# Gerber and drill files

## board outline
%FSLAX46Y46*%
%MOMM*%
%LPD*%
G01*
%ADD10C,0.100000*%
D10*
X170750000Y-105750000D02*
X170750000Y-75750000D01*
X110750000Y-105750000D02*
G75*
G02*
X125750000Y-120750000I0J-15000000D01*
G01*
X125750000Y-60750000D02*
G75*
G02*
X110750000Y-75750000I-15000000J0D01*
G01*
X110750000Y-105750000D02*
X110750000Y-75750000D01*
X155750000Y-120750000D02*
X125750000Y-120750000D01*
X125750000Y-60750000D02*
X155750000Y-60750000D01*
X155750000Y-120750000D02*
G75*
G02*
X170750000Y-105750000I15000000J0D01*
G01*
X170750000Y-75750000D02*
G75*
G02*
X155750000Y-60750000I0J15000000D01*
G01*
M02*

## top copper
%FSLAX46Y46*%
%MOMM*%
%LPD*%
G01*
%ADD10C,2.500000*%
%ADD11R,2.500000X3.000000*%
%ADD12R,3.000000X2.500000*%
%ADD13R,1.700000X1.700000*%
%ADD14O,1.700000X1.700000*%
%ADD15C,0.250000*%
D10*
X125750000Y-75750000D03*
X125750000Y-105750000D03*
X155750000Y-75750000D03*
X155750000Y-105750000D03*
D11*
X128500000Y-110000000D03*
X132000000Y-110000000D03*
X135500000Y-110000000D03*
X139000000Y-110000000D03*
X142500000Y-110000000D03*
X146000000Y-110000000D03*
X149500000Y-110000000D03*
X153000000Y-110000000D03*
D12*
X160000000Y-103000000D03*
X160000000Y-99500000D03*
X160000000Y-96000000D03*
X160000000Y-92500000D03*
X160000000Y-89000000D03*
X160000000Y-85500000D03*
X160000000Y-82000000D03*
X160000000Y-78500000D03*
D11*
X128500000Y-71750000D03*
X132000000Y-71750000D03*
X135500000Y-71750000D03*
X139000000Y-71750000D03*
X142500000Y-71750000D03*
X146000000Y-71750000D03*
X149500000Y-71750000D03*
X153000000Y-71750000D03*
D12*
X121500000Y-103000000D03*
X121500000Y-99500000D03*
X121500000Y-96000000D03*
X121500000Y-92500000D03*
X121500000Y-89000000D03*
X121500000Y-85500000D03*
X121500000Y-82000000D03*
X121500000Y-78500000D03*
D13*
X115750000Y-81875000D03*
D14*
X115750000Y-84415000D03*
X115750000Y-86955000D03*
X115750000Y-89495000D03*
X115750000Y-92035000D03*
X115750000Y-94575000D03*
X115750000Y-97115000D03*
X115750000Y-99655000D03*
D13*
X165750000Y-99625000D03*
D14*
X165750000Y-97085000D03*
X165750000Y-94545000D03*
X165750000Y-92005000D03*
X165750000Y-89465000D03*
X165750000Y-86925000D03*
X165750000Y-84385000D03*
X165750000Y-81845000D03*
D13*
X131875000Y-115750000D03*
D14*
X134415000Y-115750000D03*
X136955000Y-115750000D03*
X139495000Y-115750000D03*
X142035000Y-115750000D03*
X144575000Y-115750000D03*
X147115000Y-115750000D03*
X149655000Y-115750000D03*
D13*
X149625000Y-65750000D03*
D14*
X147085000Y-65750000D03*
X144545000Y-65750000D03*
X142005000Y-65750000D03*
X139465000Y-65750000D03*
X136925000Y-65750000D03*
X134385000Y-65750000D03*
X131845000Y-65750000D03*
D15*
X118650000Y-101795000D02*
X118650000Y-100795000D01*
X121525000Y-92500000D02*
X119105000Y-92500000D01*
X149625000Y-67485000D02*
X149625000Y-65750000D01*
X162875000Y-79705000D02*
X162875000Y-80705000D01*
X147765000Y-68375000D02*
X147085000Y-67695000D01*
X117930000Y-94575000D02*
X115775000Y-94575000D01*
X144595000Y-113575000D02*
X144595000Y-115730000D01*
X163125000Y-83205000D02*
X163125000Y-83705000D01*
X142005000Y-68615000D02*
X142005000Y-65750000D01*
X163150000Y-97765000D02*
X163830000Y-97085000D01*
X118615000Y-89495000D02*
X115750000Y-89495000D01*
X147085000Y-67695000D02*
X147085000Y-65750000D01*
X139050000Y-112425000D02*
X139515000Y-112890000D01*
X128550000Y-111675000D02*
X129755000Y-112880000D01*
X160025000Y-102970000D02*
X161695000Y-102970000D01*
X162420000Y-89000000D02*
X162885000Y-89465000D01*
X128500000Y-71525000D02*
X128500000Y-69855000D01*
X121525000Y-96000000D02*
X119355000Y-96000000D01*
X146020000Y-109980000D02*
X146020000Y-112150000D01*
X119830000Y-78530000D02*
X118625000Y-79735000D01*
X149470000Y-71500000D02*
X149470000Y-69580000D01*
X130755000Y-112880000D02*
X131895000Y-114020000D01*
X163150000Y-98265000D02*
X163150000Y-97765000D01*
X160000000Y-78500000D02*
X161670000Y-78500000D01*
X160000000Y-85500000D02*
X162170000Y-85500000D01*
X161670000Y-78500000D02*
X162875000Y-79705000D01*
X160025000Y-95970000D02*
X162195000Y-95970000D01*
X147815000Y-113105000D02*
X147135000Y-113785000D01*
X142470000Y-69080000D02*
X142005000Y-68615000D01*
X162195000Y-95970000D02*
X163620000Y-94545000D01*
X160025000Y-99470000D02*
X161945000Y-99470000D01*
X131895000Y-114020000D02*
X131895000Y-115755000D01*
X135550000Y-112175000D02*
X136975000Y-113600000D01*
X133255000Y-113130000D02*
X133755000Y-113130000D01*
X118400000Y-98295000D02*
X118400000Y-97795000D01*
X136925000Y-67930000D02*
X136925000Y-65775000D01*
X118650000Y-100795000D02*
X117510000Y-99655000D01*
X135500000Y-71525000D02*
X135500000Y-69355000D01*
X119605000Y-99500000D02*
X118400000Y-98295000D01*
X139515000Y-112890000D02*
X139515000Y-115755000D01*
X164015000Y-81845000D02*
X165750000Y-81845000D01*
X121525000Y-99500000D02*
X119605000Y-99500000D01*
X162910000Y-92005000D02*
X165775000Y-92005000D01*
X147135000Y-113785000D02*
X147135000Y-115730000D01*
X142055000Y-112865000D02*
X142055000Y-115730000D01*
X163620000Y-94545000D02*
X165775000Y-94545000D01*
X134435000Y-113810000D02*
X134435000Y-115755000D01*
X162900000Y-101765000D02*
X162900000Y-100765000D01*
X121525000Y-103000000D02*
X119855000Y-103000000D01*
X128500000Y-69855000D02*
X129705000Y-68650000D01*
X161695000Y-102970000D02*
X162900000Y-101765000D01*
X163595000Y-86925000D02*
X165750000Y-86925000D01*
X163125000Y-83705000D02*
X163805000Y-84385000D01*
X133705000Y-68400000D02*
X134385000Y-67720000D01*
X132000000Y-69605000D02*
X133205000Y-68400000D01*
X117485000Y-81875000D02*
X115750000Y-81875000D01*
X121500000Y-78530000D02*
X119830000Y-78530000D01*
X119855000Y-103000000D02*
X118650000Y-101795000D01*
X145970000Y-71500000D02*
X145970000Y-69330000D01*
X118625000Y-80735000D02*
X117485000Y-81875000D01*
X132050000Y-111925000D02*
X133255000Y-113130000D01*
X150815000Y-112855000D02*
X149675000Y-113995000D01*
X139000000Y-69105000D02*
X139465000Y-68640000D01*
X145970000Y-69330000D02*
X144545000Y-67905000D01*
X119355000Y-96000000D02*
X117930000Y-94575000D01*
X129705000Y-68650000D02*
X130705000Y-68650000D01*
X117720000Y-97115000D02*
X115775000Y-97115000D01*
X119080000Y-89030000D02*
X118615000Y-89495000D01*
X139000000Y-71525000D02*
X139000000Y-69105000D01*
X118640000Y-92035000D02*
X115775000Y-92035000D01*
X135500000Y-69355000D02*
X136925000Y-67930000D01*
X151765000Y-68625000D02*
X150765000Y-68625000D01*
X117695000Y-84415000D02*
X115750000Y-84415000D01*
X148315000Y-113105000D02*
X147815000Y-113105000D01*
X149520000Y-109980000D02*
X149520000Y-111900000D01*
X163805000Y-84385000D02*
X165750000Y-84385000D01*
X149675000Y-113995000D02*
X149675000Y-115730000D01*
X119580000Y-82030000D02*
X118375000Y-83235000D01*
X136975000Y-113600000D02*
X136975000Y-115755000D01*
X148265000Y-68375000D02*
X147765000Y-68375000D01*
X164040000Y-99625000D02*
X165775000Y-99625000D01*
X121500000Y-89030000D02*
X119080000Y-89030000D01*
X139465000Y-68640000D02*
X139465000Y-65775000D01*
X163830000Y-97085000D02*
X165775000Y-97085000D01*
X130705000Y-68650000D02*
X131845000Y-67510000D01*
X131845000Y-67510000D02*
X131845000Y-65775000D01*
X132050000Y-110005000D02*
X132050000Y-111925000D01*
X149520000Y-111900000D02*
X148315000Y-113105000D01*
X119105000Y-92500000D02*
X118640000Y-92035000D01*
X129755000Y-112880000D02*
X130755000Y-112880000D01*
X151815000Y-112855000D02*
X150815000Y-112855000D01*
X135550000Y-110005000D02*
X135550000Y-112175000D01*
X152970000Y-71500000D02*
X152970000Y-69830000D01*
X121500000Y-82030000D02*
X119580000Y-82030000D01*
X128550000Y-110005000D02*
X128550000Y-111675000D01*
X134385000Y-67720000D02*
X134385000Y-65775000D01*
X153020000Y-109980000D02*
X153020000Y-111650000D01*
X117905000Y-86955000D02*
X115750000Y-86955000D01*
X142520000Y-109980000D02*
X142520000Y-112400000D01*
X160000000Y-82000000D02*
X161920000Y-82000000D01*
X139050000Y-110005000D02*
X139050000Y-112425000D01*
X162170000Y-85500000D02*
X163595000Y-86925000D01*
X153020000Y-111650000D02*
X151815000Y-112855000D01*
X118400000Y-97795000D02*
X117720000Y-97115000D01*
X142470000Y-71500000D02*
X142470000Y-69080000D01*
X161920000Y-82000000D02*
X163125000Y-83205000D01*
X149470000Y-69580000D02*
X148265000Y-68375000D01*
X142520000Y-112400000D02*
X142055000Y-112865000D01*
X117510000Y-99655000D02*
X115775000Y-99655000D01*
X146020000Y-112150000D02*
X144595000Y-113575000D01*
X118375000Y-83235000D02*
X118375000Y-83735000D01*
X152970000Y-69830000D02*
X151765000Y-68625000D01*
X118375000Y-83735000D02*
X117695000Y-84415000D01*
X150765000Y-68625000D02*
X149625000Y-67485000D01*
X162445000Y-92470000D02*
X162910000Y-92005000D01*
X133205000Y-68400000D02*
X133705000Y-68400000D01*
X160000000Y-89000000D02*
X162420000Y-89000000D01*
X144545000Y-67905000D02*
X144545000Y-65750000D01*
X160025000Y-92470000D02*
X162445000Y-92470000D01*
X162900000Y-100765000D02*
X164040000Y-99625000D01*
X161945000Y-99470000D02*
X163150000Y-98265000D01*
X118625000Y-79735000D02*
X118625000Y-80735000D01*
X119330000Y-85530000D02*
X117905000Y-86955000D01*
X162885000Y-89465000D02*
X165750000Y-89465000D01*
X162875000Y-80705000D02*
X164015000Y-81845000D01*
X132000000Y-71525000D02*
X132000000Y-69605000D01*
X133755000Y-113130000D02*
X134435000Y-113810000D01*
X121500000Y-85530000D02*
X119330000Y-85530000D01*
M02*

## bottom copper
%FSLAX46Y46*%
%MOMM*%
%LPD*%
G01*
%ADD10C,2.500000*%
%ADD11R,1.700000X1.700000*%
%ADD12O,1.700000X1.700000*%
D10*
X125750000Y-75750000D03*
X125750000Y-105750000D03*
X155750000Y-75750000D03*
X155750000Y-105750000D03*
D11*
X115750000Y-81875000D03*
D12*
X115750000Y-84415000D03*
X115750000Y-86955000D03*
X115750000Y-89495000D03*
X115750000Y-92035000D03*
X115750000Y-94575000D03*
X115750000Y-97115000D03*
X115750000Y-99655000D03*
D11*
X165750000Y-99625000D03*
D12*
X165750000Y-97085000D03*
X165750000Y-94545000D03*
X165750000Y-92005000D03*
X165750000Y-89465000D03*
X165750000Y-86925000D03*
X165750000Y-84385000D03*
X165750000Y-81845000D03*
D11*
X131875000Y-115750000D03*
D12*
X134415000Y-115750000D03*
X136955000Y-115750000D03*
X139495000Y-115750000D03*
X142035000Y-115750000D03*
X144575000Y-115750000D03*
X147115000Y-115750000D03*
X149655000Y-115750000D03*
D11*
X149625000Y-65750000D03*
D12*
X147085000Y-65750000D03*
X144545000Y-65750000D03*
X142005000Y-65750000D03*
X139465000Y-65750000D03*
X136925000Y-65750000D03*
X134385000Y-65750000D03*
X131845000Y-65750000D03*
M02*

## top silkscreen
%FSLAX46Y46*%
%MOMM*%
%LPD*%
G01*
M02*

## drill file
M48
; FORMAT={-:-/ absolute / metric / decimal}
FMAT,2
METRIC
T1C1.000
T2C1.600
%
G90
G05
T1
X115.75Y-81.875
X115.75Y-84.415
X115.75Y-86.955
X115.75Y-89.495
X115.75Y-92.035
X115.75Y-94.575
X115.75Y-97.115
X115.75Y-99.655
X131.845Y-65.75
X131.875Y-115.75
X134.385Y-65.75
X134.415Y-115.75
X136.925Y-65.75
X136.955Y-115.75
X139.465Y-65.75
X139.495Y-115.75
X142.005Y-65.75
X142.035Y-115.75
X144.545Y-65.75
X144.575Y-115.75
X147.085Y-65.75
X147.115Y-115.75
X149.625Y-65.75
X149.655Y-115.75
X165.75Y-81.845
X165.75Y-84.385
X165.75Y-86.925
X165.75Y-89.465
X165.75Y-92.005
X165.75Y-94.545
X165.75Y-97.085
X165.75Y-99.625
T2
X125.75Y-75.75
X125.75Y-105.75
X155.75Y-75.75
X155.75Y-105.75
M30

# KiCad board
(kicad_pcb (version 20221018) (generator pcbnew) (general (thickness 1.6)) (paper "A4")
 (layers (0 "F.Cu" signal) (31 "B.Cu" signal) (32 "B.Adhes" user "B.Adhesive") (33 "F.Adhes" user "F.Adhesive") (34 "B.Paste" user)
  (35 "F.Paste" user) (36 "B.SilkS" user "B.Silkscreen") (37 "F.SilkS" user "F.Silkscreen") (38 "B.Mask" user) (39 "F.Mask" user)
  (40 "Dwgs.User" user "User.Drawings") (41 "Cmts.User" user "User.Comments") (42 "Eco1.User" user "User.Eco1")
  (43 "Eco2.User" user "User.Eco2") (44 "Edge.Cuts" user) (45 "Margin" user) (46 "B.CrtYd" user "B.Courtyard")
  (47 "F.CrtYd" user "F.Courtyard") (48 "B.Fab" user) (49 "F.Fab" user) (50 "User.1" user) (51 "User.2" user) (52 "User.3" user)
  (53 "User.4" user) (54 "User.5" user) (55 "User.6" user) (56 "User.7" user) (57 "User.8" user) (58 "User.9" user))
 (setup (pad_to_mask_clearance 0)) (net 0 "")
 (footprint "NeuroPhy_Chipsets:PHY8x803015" (layer "F.Cu") (at 140.75 90.75)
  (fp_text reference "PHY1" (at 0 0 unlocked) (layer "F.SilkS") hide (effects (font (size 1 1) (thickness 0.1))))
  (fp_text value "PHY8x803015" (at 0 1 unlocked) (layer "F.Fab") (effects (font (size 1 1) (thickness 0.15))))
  (pad "" thru_hole circle (at -15 -15 90) (size 2.5 2.5) (drill 1.6) (layers "*.Cu" "*.Mask"))
  (pad "" thru_hole circle (at -15 15 90) (size 2.5 2.5) (drill 1.6) (layers "*.Cu" "*.Mask"))
  (pad "" thru_hole circle (at 15 -15 90) (size 2.5 2.5) (drill 1.6) (layers "*.Cu" "*.Mask"))
  (pad "" thru_hole circle (at 15 15 90) (size 2.5 2.5) (drill 1.6) (layers "*.Cu" "*.Mask"))
  (pad "1" smd rect (at -12.25 19.25 90) (size 3 2.5) (layers "F.Cu" "F.Paste" "F.Mask"))
  (pad "2" smd rect (at -8.75 19.25 90) (size 3 2.5) (layers "F.Cu" "F.Paste" "F.Mask"))
  (pad "3" smd rect (at -5.25 19.25 90) (size 3 2.5) (layers "F.Cu" "F.Paste" "F.Mask"))
  (pad "4" smd rect (at -1.75 19.25 90) (size 3 2.5) (layers "F.Cu" "F.Paste" "F.Mask"))
  (pad "5" smd rect (at 1.75 19.25 90) (size 3 2.5) (layers "F.Cu" "F.Paste" "F.Mask"))
  (pad "6" smd rect (at 5.25 19.25 90) (size 3 2.5) (layers "F.Cu" "F.Paste" "F.Mask"))
  (pad "7" smd rect (at 8.75 19.25 90) (size 3 2.5) (layers "F.Cu" "F.Paste" "F.Mask"))
  (pad "8" smd rect (at 12.25 19.25 90) (size 3 2.5) (layers "F.Cu" "F.Paste" "F.Mask"))
  (pad "9" smd rect (at 19.25 12.25 180) (size 3 2.5) (layers "F.Cu" "F.Paste" "F.Mask"))
  (pad "10" smd rect (at 19.25 8.75 180) (size 3 2.5) (layers "F.Cu" "F.Paste" "F.Mask"))
  (pad "11" smd rect (at 19.25 5.25 180) (size 3 2.5) (layers "F.Cu" "F.Paste" "F.Mask"))
  (pad "12" smd rect (at 19.25 1.75 180) (size 3 2.5) (layers "F.Cu" "F.Paste" "F.Mask"))
  (pad "13" smd rect (at 19.25 -1.75 180) (size 3 2.5) (layers "F.Cu" "F.Paste" "F.Mask"))
  (pad "14" smd rect (at 19.25 -5.25 180) (size 3 2.5) (layers "F.Cu" "F.Paste" "F.Mask"))
  (pad "15" smd rect (at 19.25 -8.75 180) (size 3 2.5) (layers "F.Cu" "F.Paste" "F.Mask"))
  (pad "16" smd rect (at 19.25 -12.25 180) (size 3 2.5) (layers "F.Cu" "F.Paste" "F.Mask"))
  (pad "17" smd rect (at -12.25 -19 90) (size 3 2.5) (layers "F.Cu" "F.Paste" "F.Mask"))
  (pad "18" smd rect (at -8.75 -19 90) (size 3 2.5) (layers "F.Cu" "F.Paste" "F.Mask"))
  (pad "19" smd rect (at -5.25 -19 90) (size 3 2.5) (layers "F.Cu" "F.Paste" "F.Mask"))
  (pad "20" smd rect (at -1.75 -19 90) (size 3 2.5) (layers "F.Cu" "F.Paste" "F.Mask"))
  (pad "21" smd rect (at 1.75 -19 90) (size 3 2.5) (layers "F.Cu" "F.Paste" "F.Mask"))
  (pad "22" smd rect (at 5.25 -19 90) (size 3 2.5) (layers "F.Cu" "F.Paste" "F.Mask"))
  (pad "23" smd rect (at 8.75 -19 90) (size 3 2.5) (layers "F.Cu" "F.Paste" "F.Mask"))
  (pad "24" smd rect (at 12.25 -19 90) (size 3 2.5) (layers "F.Cu" "F.Paste" "F.Mask"))
  (pad "25" smd rect (at -19.25 12.25 180) (size 3 2.5) (layers "F.Cu" "F.Paste" "F.Mask"))
  (pad "26" smd rect (at -19.25 8.75 180) (size 3 2.5) (layers "F.Cu" "F.Paste" "F.Mask"))
  (pad "27" smd rect (at -19.25 5.25 180) (size 3 2.5) (layers "F.Cu" "F.Paste" "F.Mask"))
  (pad "28" smd rect (at -19.25 1.75 180) (size 3 2.5) (layers "F.Cu" "F.Paste" "F.Mask"))
  (pad "29" smd rect (at -19.25 -1.75 180) (size 3 2.5) (layers "F.Cu" "F.Paste" "F.Mask"))
  (pad "30" smd rect (at -19.25 -5.25 180) (size 3 2.5) (layers "F.Cu" "F.Paste" "F.Mask"))
  (pad "31" smd rect (at -19.25 -8.75 180) (size 3 2.5) (layers "F.Cu" "F.Paste" "F.Mask"))
  (pad "32" smd rect (at -19.25 -12.25 180) (size 3 2.5) (layers "F.Cu" "F.Paste" "F.Mask")))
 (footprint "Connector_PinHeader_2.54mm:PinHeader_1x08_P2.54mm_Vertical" (layer "B.Cu") (at 115.75 81.875 180)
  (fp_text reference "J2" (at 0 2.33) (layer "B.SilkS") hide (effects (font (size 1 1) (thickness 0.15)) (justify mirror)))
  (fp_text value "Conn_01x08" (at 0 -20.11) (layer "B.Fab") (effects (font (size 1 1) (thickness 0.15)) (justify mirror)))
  (pad "1" thru_hole rect (at 0 0 180) (size 1.7 1.7) (drill 1) (layers "*.Cu" "*.Mask"))
  (pad "2" thru_hole oval (at 0 -2.54 180) (size 1.7 1.7) (drill 1) (layers "*.Cu" "*.Mask"))
  (pad "3" thru_hole oval (at 0 -5.08 180) (size 1.7 1.7) (drill 1) (layers "*.Cu" "*.Mask"))
  (pad "4" thru_hole oval (at 0 -7.62 180) (size 1.7 1.7) (drill 1) (layers "*.Cu" "*.Mask"))
  (pad "5" thru_hole oval (at 0 -10.16 180) (size 1.7 1.7) (drill 1) (layers "*.Cu" "*.Mask"))
  (pad "6" thru_hole oval (at 0 -12.7 180) (size 1.7 1.7) (drill 1) (layers "*.Cu" "*.Mask"))
  (pad "7" thru_hole oval (at 0 -15.24 180) (size 1.7 1.7) (drill 1) (layers "*.Cu" "*.Mask"))
  (pad "8" thru_hole oval (at 0 -17.78 180) (size 1.7 1.7) (drill 1) (layers "*.Cu" "*.Mask")))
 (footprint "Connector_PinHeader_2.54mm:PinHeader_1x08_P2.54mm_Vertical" (layer "B.Cu") (at 165.75 99.625)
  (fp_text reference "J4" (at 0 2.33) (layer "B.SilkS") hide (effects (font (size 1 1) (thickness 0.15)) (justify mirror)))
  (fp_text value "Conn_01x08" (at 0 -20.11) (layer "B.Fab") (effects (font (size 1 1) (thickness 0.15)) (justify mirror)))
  (pad "1" thru_hole rect (at 0 0) (size 1.7 1.7) (drill 1) (layers "*.Cu" "*.Mask"))
  (pad "2" thru_hole oval (at 0 -2.54) (size 1.7 1.7) (drill 1) (layers "*.Cu" "*.Mask"))
  (pad "3" thru_hole oval (at 0 -5.08) (size 1.7 1.7) (drill 1) (layers "*.Cu" "*.Mask"))
  (pad "4" thru_hole oval (at 0 -7.62) (size 1.7 1.7) (drill 1) (layers "*.Cu" "*.Mask"))
  (pad "5" thru_hole oval (at 0 -10.16) (size 1.7 1.7) (drill 1) (layers "*.Cu" "*.Mask"))
  (pad "6" thru_hole oval (at 0 -12.7) (size 1.7 1.7) (drill 1) (layers "*.Cu" "*.Mask"))
  (pad "7" thru_hole oval (at 0 -15.24) (size 1.7 1.7) (drill 1) (layers "*.Cu" "*.Mask"))
  (pad "8" thru_hole oval (at 0 -17.78) (size 1.7 1.7) (drill 1) (layers "*.Cu" "*.Mask")))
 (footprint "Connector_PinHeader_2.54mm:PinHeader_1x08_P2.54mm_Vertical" (layer "B.Cu") (at 131.875 115.75 -90)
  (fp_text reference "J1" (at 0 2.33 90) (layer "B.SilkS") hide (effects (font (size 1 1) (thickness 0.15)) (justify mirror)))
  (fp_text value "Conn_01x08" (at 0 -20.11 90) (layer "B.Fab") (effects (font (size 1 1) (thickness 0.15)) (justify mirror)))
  (pad "1" thru_hole rect (at 0 0 270) (size 1.7 1.7) (drill 1) (layers "*.Cu" "*.Mask"))
  (pad "2" thru_hole oval (at 0 -2.54 270) (size 1.7 1.7) (drill 1) (layers "*.Cu" "*.Mask"))
  (pad "3" thru_hole oval (at 0 -5.08 270) (size 1.7 1.7) (drill 1) (layers "*.Cu" "*.Mask"))
  (pad "4" thru_hole oval (at 0 -7.62 270) (size 1.7 1.7) (drill 1) (layers "*.Cu" "*.Mask"))
  (pad "5" thru_hole oval (at 0 -10.16 270) (size 1.7 1.7) (drill 1) (layers "*.Cu" "*.Mask"))
  (pad "6" thru_hole oval (at 0 -12.7 270) (size 1.7 1.7) (drill 1) (layers "*.Cu" "*.Mask"))
  (pad "7" thru_hole oval (at 0 -15.24 270) (size 1.7 1.7) (drill 1) (layers "*.Cu" "*.Mask"))
  (pad "8" thru_hole oval (at 0 -17.78 270) (size 1.7 1.7) (drill 1) (layers "*.Cu" "*.Mask")))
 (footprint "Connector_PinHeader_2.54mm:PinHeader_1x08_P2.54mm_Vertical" (layer "B.Cu") (at 149.625 65.75 90)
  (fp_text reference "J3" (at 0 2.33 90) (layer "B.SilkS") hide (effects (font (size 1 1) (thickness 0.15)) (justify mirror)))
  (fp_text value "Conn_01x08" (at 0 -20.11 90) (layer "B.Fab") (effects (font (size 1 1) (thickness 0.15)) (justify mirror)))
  (pad "1" thru_hole rect (at 0 0 90) (size 1.7 1.7) (drill 1) (layers "*.Cu" "*.Mask"))
  (pad "2" thru_hole oval (at 0 -2.54 90) (size 1.7 1.7) (drill 1) (layers "*.Cu" "*.Mask"))
  (pad "3" thru_hole oval (at 0 -5.08 90) (size 1.7 1.7) (drill 1) (layers "*.Cu" "*.Mask"))
  (pad "4" thru_hole oval (at 0 -7.62 90) (size 1.7 1.7) (drill 1) (layers "*.Cu" "*.Mask"))
  (pad "5" thru_hole oval (at 0 -10.16 90) (size 1.7 1.7) (drill 1) (layers "*.Cu" "*.Mask"))
  (pad "6" thru_hole oval (at 0 -12.7 90) (size 1.7 1.7) (drill 1) (layers "*.Cu" "*.Mask"))
  (pad "7" thru_hole oval (at 0 -15.24 90) (size 1.7 1.7) (drill 1) (layers "*.Cu" "*.Mask"))
  (pad "8" thru_hole oval (at 0 -17.78 90) (size 1.7 1.7) (drill 1) (layers "*.Cu" "*.Mask")))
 (gr_line (start 170.75 105.75) (end 170.75 75.75) (stroke (width 0.1) (type default)) (layer "Edge.Cuts"))
 (gr_arc (start 110.75 105.75) (mid 121.356602 110.143398) (end 125.75 120.75) (stroke (width 0.1) (type default)) (layer "Edge.Cuts"))
 (gr_arc (start 125.75 60.75) (mid 121.356602 71.356602) (end 110.75 75.75) (stroke (width 0.1) (type default)) (layer "Edge.Cuts"))
 (gr_line (start 110.75 105.75) (end 110.75 75.75) (stroke (width 0.1) (type default)) (layer "Edge.Cuts"))
 (gr_line (start 155.75 120.75) (end 125.75 120.75) (stroke (width 0.1) (type default)) (layer "Edge.Cuts"))
 (gr_line (start 125.75 60.75) (end 155.75 60.75) (stroke (width 0.1) (type default)) (layer "Edge.Cuts"))
 (gr_arc (start 155.75 120.75) (mid 160.143398 110.143398) (end 170.75 105.75) (stroke (width 0.1) (type default)) (layer "Edge.Cuts"))
 (gr_arc (start 170.75 75.75) (mid 160.143398 71.356602) (end 155.75 60.75) (stroke (width 0.1) (type default)) (layer "Edge.Cuts"))
 (segment (start 118.65 101.795) (end 118.65 100.795) (width 0.25) (layer "F.Cu") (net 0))
 (segment (start 121.525 92.5) (end 119.105 92.5) (width 0.25) (layer "F.Cu") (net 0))
 (segment (start 149.625 67.485) (end 149.625 65.75) (width 0.25) (layer "F.Cu") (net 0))
 (segment (start 162.875 79.705) (end 162.875 80.705) (width 0.25) (layer "F.Cu") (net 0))
 (segment (start 147.765 68.375) (end 147.085 67.695) (width 0.25) (layer "F.Cu") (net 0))
 (segment (start 117.93 94.575) (end 115.775 94.575) (width 0.25) (layer "F.Cu") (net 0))
 (segment (start 144.595 113.575) (end 144.595 115.73) (width 0.25) (layer "F.Cu") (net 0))
 (segment (start 163.125 83.205) (end 163.125 83.705) (width 0.25) (layer "F.Cu") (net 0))
 (segment (start 142.005 68.615) (end 142.005 65.75) (width 0.25) (layer "F.Cu") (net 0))
 (segment (start 163.15 97.765) (end 163.83 97.085) (width 0.25) (layer "F.Cu") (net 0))
 (segment (start 118.615 89.495) (end 115.75 89.495) (width 0.25) (layer "F.Cu") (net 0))
 (segment (start 147.085 67.695) (end 147.085 65.75) (width 0.25) (layer "F.Cu") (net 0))
 (segment (start 139.05 112.425) (end 139.515 112.89) (width 0.25) (layer "F.Cu") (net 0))
 (segment (start 128.55 111.675) (end 129.755 112.88) (width 0.25) (layer "F.Cu") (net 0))
 (segment (start 160.025 102.97) (end 161.695 102.97) (width 0.25) (layer "F.Cu") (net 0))
 (segment (start 162.42 89) (end 162.885 89.465) (width 0.25) (layer "F.Cu") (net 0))
 (segment (start 128.5 71.525) (end 128.5 69.855) (width 0.25) (layer "F.Cu") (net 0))
 (segment (start 121.525 96) (end 119.355 96) (width 0.25) (layer "F.Cu") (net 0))
 (segment (start 146.02 109.98) (end 146.02 112.15) (width 0.25) (layer "F.Cu") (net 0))
 (segment (start 119.83 78.53) (end 118.625 79.735) (width 0.25) (layer "F.Cu") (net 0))
 (segment (start 149.47 71.5) (end 149.47 69.58) (width 0.25) (layer "F.Cu") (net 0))
 (segment (start 130.755 112.88) (end 131.895 114.02) (width 0.25) (layer "F.Cu") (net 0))
 (segment (start 163.15 98.265) (end 163.15 97.765) (width 0.25) (layer "F.Cu") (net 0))
 (segment (start 160 78.5) (end 161.67 78.5) (width 0.25) (layer "F.Cu") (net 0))
 (segment (start 160 85.5) (end 162.17 85.5) (width 0.25) (layer "F.Cu") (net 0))
 (segment (start 161.67 78.5) (end 162.875 79.705) (width 0.25) (layer "F.Cu") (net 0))
 (segment (start 160.025 95.97) (end 162.195 95.97) (width 0.25) (layer "F.Cu") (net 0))
 (segment (start 147.815 113.105) (end 147.135 113.785) (width 0.25) (layer "F.Cu") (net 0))
 (segment (start 142.47 69.08) (end 142.005 68.615) (width 0.25) (layer "F.Cu") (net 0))
 (segment (start 162.195 95.97) (end 163.62 94.545) (width 0.25) (layer "F.Cu") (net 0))
 (segment (start 160.025 99.47) (end 161.945 99.47) (width 0.25) (layer "F.Cu") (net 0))
 (segment (start 131.895 114.02) (end 131.895 115.755) (width 0.25) (layer "F.Cu") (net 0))
 (segment (start 135.55 112.175) (end 136.975 113.6) (width 0.25) (layer "F.Cu") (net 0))
 (segment (start 133.255 113.13) (end 133.755 113.13) (width 0.25) (layer "F.Cu") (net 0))
 (segment (start 118.4 98.295) (end 118.4 97.795) (width 0.25) (layer "F.Cu") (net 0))
 (segment (start 136.925 67.93) (end 136.925 65.775) (width 0.25) (layer "F.Cu") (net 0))
 (segment (start 118.65 100.795) (end 117.51 99.655) (width 0.25) (layer "F.Cu") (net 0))
 (segment (start 135.5 71.525) (end 135.5 69.355) (width 0.25) (layer "F.Cu") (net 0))
 (segment (start 119.605 99.5) (end 118.4 98.295) (width 0.25) (layer "F.Cu") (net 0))
 (segment (start 139.515 112.89) (end 139.515 115.755) (width 0.25) (layer "F.Cu") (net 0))
 (segment (start 164.015 81.845) (end 165.75 81.845) (width 0.25) (layer "F.Cu") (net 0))
 (segment (start 121.525 99.5) (end 119.605 99.5) (width 0.25) (layer "F.Cu") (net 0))
 (segment (start 162.91 92.005) (end 165.775 92.005) (width 0.25) (layer "F.Cu") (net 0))
 (segment (start 147.135 113.785) (end 147.135 115.73) (width 0.25) (layer "F.Cu") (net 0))
 (segment (start 142.055 112.865) (end 142.055 115.73) (width 0.25) (layer "F.Cu") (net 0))
 (segment (start 163.62 94.545) (end 165.775 94.545) (width 0.25) (layer "F.Cu") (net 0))
 (segment (start 134.435 113.81) (end 134.435 115.755) (width 0.25) (layer "F.Cu") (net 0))
 (segment (start 162.9 101.765) (end 162.9 100.765) (width 0.25) (layer "F.Cu") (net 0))
 (segment (start 121.525 103) (end 119.855 103) (width 0.25) (layer "F.Cu") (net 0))
 (segment (start 128.5 69.855) (end 129.705 68.65) (width 0.25) (layer "F.Cu") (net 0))
 (segment (start 161.695 102.97) (end 162.9 101.765) (width 0.25) (layer "F.Cu") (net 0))
 (segment (start 163.595 86.925) (end 165.75 86.925) (width 0.25) (layer "F.Cu") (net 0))
 (segment (start 163.125 83.705) (end 163.805 84.385) (width 0.25) (layer "F.Cu") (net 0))
 (segment (start 133.705 68.4) (end 134.385 67.72) (width 0.25) (layer "F.Cu") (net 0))
 (segment (start 132 69.605) (end 133.205 68.4) (width 0.25) (layer "F.Cu") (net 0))
 (segment (start 117.485 81.875) (end 115.75 81.875) (width 0.25) (layer "F.Cu") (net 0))
 (segment (start 121.5 78.53) (end 119.83 78.53) (width 0.25) (layer "F.Cu") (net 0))
 (segment (start 119.855 103) (end 118.65 101.795) (width 0.25) (layer "F.Cu") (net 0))
 (segment (start 145.97 71.5) (end 145.97 69.33) (width 0.25) (layer "F.Cu") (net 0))
 (segment (start 118.625 80.735) (end 117.485 81.875) (width 0.25) (layer "F.Cu") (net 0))
 (segment (start 132.05 111.925) (end 133.255 113.13) (width 0.25) (layer "F.Cu") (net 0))
 (segment (start 150.815 112.855) (end 149.675 113.995) (width 0.25) (layer "F.Cu") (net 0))
 (segment (start 139 69.105) (end 139.465 68.64) (width 0.25) (layer "F.Cu") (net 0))
 (segment (start 145.97 69.33) (end 144.545 67.905) (width 0.25) (layer "F.Cu") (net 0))
 (segment (start 119.355 96) (end 117.93 94.575) (width 0.25) (layer "F.Cu") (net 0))
 (segment (start 129.705 68.65) (end 130.705 68.65) (width 0.25) (layer "F.Cu") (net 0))
 (segment (start 117.72 97.115) (end 115.775 97.115) (width 0.25) (layer "F.Cu") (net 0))
 (segment (start 119.08 89.03) (end 118.615 89.495) (width 0.25) (layer "F.Cu") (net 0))
 (segment (start 139 71.525) (end 139 69.105) (width 0.25) (layer "F.Cu") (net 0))
 (segment (start 118.64 92.035) (end 115.775 92.035) (width 0.25) (layer "F.Cu") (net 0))
 (segment (start 135.5 69.355) (end 136.925 67.93) (width 0.25) (layer "F.Cu") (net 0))
 (segment (start 151.765 68.625) (end 150.765 68.625) (width 0.25) (layer "F.Cu") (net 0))
 (segment (start 117.695 84.415) (end 115.75 84.415) (width 0.25) (layer "F.Cu") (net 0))
 (segment (start 148.315 113.105) (end 147.815 113.105) (width 0.25) (layer "F.Cu") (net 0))
 (segment (start 149.52 109.98) (end 149.52 111.9) (width 0.25) (layer "F.Cu") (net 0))
 (segment (start 163.805 84.385) (end 165.75 84.385) (width 0.25) (layer "F.Cu") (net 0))
 (segment (start 149.675 113.995) (end 149.675 115.73) (width 0.25) (layer "F.Cu") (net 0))
 (segment (start 119.58 82.03) (end 118.375 83.235) (width 0.25) (layer "F.Cu") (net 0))
 (segment (start 136.975 113.6) (end 136.975 115.755) (width 0.25) (layer "F.Cu") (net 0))
 (segment (start 148.265 68.375) (end 147.765 68.375) (width 0.25) (layer "F.Cu") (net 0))
 (segment (start 164.04 99.625) (end 165.775 99.625) (width 0.25) (layer "F.Cu") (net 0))
 (segment (start 121.5 89.03) (end 119.08 89.03) (width 0.25) (layer "F.Cu") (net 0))
 (segment (start 139.465 68.64) (end 139.465 65.775) (width 0.25) (layer "F.Cu") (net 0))
 (segment (start 163.83 97.085) (end 165.775 97.085) (width 0.25) (layer "F.Cu") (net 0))
 (segment (start 130.705 68.65) (end 131.845 67.51) (width 0.25) (layer "F.Cu") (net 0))
 (segment (start 131.845 67.51) (end 131.845 65.775) (width 0.25) (layer "F.Cu") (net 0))
 (segment (start 132.05 110.005) (end 132.05 111.925) (width 0.25) (layer "F.Cu") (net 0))
 (segment (start 149.52 111.9) (end 148.315 113.105) (width 0.25) (layer "F.Cu") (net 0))
 (segment (start 119.105 92.5) (end 118.64 92.035) (width 0.25) (layer "F.Cu") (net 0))
 (segment (start 129.755 112.88) (end 130.755 112.88) (width 0.25) (layer "F.Cu") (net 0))
 (segment (start 151.815 112.855) (end 150.815 112.855) (width 0.25) (layer "F.Cu") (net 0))
 (segment (start 135.55 110.005) (end 135.55 112.175) (width 0.25) (layer "F.Cu") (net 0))
 (segment (start 152.97 71.5) (end 152.97 69.83) (width 0.25) (layer "F.Cu") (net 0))
 (segment (start 121.5 82.03) (end 119.58 82.03) (width 0.25) (layer "F.Cu") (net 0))
 (segment (start 128.55 110.005) (end 128.55 111.675) (width 0.25) (layer "F.Cu") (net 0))
 (segment (start 134.385 67.72) (end 134.385 65.775) (width 0.25) (layer "F.Cu") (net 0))
 (segment (start 153.02 109.98) (end 153.02 111.65) (width 0.25) (layer "F.Cu") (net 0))
 (segment (start 117.905 86.955) (end 115.75 86.955) (width 0.25) (layer "F.Cu") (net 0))
 (segment (start 142.52 109.98) (end 142.52 112.4) (width 0.25) (layer "F.Cu") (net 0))
 (segment (start 160 82) (end 161.92 82) (width 0.25) (layer "F.Cu") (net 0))
 (segment (start 139.05 110.005) (end 139.05 112.425) (width 0.25) (layer "F.Cu") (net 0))
 (segment (start 162.17 85.5) (end 163.595 86.925) (width 0.25) (layer "F.Cu") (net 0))
 (segment (start 153.02 111.65) (end 151.815 112.855) (width 0.25) (layer "F.Cu") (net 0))
 (segment (start 118.4 97.795) (end 117.72 97.115) (width 0.25) (layer "F.Cu") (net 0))
 (segment (start 142.47 71.5) (end 142.47 69.08) (width 0.25) (layer "F.Cu") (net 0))
 (segment (start 161.92 82) (end 163.125 83.205) (width 0.25) (layer "F.Cu") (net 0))
 (segment (start 149.47 69.58) (end 148.265 68.375) (width 0.25) (layer "F.Cu") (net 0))
 (segment (start 142.52 112.4) (end 142.055 112.865) (width 0.25) (layer "F.Cu") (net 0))
 (segment (start 117.51 99.655) (end 115.775 99.655) (width 0.25) (layer "F.Cu") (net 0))
 (segment (start 146.02 112.15) (end 144.595 113.575) (width 0.25) (layer "F.Cu") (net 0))
 (segment (start 118.375 83.235) (end 118.375 83.735) (width 0.25) (layer "F.Cu") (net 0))
 (segment (start 152.97 69.83) (end 151.765 68.625) (width 0.25) (layer "F.Cu") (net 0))
 (segment (start 118.375 83.735) (end 117.695 84.415) (width 0.25) (layer "F.Cu") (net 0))
 (segment (start 150.765 68.625) (end 149.625 67.485) (width 0.25) (layer "F.Cu") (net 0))
 (segment (start 162.445 92.47) (end 162.91 92.005) (width 0.25) (layer "F.Cu") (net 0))
 (segment (start 133.205 68.4) (end 133.705 68.4) (width 0.25) (layer "F.Cu") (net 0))
 (segment (start 160 89) (end 162.42 89) (width 0.25) (layer "F.Cu") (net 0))
 (segment (start 144.545 67.905) (end 144.545 65.75) (width 0.25) (layer "F.Cu") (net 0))
 (segment (start 160.025 92.47) (end 162.445 92.47) (width 0.25) (layer "F.Cu") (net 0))
 (segment (start 162.9 100.765) (end 164.04 99.625) (width 0.25) (layer "F.Cu") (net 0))
 (segment (start 161.945 99.47) (end 163.15 98.265) (width 0.25) (layer "F.Cu") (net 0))
 (segment (start 118.625 79.735) (end 118.625 80.735) (width 0.25) (layer "F.Cu") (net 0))
 (segment (start 119.33 85.53) (end 117.905 86.955) (width 0.25) (layer "F.Cu") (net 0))
 (segment (start 162.885 89.465) (end 165.75 89.465) (width 0.25) (layer "F.Cu") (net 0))
 (segment (start 162.875 80.705) (end 164.015 81.845) (width 0.25) (layer "F.Cu") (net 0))
 (segment (start 132 71.525) (end 132 69.605) (width 0.25) (layer "F.Cu") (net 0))
 (segment (start 133.755 113.13) (end 134.435 113.81) (width 0.25) (layer "F.Cu") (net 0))
 (segment (start 121.5 85.53) (end 119.33 85.53) (width 0.25) (layer "F.Cu") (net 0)))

